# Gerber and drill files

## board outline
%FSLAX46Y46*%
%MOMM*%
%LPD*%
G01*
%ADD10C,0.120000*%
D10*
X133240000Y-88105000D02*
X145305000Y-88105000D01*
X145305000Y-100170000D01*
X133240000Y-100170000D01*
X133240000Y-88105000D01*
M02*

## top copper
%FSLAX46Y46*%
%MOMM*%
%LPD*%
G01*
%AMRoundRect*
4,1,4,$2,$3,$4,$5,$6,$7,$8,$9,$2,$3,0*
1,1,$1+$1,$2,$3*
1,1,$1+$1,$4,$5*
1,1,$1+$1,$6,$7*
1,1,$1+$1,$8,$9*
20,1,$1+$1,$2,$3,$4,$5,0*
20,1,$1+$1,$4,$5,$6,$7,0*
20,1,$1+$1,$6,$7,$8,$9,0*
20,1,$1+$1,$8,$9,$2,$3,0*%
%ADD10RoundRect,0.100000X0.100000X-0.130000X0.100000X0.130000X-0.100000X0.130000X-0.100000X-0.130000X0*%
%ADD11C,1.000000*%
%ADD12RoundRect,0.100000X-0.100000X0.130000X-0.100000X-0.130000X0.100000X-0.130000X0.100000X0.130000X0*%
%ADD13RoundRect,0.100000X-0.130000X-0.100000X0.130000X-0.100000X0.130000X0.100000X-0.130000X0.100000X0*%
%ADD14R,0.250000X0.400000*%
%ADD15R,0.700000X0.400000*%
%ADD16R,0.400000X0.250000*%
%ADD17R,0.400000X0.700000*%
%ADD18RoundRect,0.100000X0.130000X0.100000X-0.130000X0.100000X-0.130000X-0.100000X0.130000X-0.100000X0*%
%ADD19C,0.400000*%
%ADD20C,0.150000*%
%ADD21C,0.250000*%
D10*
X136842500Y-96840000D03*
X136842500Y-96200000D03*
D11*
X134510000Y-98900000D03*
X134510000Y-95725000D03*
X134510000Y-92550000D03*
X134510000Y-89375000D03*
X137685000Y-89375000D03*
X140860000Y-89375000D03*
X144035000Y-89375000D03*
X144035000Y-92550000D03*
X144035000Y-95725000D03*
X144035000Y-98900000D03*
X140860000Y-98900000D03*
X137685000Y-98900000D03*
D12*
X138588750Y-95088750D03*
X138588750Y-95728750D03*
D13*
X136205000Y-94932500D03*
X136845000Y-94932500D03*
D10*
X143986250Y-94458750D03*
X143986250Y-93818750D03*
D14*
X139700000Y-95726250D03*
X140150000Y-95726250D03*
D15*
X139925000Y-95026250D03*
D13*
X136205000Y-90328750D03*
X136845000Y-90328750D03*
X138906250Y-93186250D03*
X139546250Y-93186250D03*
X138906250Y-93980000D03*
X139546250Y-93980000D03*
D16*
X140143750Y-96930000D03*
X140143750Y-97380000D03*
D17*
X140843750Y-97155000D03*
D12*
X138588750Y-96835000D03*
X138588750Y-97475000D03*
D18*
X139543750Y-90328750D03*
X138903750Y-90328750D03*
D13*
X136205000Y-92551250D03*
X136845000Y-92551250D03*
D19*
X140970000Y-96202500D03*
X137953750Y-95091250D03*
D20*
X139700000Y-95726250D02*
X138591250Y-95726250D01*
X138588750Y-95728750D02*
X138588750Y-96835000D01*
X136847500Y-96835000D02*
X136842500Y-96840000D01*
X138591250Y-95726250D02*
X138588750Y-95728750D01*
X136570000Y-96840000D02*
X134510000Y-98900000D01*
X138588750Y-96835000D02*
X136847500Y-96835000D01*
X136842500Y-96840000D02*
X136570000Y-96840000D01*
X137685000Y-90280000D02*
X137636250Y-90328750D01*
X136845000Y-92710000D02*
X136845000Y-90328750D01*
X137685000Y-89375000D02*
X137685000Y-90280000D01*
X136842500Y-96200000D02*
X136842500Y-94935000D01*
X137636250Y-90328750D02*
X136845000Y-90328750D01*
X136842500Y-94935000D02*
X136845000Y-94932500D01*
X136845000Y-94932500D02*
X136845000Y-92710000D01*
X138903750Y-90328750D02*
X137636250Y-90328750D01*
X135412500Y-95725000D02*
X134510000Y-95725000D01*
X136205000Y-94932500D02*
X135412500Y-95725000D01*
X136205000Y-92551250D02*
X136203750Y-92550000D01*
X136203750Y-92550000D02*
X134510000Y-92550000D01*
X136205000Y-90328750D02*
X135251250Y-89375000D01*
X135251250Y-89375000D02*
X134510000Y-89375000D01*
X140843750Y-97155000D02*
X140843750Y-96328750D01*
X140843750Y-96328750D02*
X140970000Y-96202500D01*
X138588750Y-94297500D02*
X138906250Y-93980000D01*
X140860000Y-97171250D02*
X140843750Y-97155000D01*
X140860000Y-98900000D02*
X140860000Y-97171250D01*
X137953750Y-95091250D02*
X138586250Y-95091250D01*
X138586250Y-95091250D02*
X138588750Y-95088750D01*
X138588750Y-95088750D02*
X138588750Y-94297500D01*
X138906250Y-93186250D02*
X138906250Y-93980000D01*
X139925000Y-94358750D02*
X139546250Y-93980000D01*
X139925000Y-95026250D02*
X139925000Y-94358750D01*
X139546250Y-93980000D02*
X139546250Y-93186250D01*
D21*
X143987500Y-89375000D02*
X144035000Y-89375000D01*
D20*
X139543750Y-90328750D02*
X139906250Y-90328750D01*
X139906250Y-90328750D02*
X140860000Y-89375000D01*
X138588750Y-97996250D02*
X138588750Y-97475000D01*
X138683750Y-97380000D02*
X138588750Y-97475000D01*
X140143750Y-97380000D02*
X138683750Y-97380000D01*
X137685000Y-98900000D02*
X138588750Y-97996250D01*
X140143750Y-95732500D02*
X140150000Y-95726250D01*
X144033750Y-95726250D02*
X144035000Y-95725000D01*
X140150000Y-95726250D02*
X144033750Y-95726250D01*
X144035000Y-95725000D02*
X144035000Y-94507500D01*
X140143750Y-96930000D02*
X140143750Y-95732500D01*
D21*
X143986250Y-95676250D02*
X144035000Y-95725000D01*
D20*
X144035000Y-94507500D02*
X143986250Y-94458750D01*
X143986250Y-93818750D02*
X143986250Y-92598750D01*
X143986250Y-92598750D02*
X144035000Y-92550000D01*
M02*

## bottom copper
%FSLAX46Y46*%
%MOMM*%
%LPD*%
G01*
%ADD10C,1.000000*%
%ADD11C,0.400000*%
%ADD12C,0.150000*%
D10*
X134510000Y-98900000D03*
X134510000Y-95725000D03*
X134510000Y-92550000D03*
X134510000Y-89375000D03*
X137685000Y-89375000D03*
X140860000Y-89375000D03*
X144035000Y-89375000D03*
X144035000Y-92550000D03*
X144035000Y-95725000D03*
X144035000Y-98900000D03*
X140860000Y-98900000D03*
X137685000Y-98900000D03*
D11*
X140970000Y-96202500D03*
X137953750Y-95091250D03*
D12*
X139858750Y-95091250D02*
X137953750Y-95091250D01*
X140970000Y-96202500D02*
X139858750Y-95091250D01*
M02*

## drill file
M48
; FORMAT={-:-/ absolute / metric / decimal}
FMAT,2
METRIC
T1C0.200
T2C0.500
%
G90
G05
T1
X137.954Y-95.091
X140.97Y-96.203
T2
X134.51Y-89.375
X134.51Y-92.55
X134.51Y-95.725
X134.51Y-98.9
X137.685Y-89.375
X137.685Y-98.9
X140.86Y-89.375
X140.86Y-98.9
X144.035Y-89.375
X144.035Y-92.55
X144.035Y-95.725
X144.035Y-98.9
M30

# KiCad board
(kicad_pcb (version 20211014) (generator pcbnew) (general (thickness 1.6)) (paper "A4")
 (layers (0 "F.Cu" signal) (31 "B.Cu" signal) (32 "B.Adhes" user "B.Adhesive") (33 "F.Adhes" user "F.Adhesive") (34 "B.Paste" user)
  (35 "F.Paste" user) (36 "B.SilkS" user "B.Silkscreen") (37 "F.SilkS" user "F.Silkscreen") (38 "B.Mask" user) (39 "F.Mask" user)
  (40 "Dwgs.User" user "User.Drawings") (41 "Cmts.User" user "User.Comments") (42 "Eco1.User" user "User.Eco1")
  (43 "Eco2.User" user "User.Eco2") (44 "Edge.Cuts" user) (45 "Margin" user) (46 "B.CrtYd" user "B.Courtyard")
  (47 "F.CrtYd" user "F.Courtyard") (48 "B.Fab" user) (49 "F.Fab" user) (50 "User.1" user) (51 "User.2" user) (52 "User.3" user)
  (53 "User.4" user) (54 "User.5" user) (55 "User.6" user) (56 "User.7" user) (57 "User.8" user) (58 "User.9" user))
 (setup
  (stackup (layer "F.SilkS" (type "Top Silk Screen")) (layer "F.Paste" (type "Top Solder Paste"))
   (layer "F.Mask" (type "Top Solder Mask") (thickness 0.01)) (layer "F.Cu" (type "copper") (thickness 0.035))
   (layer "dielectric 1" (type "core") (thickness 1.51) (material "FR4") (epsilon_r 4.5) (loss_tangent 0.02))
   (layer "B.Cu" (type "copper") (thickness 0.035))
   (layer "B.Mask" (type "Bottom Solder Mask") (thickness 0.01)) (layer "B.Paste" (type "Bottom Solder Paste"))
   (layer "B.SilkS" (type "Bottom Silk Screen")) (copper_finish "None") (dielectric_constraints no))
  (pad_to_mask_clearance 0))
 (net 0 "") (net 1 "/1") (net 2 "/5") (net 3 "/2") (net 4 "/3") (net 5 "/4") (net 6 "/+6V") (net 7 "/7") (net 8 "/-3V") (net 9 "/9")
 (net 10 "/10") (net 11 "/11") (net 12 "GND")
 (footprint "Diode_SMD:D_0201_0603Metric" (layer "F.Cu") (at 136.8425 96.52 90)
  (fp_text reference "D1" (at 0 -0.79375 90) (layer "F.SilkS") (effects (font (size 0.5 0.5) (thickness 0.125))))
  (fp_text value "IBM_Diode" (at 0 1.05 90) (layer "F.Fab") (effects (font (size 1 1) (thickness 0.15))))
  (pad "" smd roundrect locked (at -0.345 0 90) (size 0.318 0.36) (layers "F.Paste") (roundrect_rratio 0.25))
  (pad "" smd roundrect locked (at 0.345 0 90) (size 0.318 0.36) (layers "F.Paste") (roundrect_rratio 0.25))
  (pad "1" smd roundrect locked (at -0.32 0 90) (size 0.46 0.4) (layers "F.Cu" "F.Mask") (roundrect_rratio 0.25) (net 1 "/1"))
  (pad "2" smd roundrect locked (at 0.32 0 90) (size 0.46 0.4) (layers "F.Cu" "F.Mask") (roundrect_rratio 0.25) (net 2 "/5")))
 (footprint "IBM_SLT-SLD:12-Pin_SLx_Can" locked (layer "F.Cu") (at 134.51 98.9)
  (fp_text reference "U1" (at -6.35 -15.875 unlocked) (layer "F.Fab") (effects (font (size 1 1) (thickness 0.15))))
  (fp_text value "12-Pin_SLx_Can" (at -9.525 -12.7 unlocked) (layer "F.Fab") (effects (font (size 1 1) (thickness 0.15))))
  (fp_rect (start -1.27 -10.795) (end 10.795 1.27) (layer "Edge.Cuts") (width 0.12) (fill none))
  (pad "1" thru_hole circle locked (at 0 0) (size 1 1) (drill 0.5) (layers *.Cu *.Mask) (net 1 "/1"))
  (pad "2" thru_hole circle locked (at 0 -3.175) (size 1 1) (drill 0.5) (layers *.Cu *.Mask) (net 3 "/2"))
  (pad "3" thru_hole circle locked (at 0 -6.35) (size 1 1) (drill 0.5) (layers *.Cu *.Mask) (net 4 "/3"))
  (pad "4" thru_hole circle locked (at 0 -9.525) (size 1 1) (drill 0.5) (layers *.Cu *.Mask) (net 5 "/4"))
  (pad "5" thru_hole circle locked (at 3.175 -9.525) (size 1 1) (drill 0.5) (layers *.Cu *.Mask) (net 2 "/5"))
  (pad "6" thru_hole circle locked (at 6.35 -9.525) (size 1 1) (drill 0.5) (layers *.Cu *.Mask) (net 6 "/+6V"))
  (pad "7" thru_hole circle locked (at 9.525 -9.525) (size 1 1) (drill 0.5) (layers *.Cu *.Mask) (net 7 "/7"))
  (pad "8" thru_hole circle locked (at 9.525 -6.35) (size 1 1) (drill 0.5) (layers *.Cu *.Mask) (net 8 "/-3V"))
  (pad "9" thru_hole circle locked (at 9.525 -3.175) (size 1 1) (drill 0.5) (layers *.Cu *.Mask) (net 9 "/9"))
  (pad "10" thru_hole circle locked (at 9.525 0) (size 1 1) (drill 0.5) (layers *.Cu *.Mask) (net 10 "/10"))
  (pad "11" thru_hole circle locked (at 6.35 0) (size 1 1) (drill 0.5) (layers *.Cu *.Mask) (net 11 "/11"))
  (pad "12" thru_hole circle locked (at 3.175 0) (size 1 1) (drill 0.5) (layers *.Cu *.Mask) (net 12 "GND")))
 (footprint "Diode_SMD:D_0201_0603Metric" (layer "F.Cu") (at 138.58875 95.40875 -90)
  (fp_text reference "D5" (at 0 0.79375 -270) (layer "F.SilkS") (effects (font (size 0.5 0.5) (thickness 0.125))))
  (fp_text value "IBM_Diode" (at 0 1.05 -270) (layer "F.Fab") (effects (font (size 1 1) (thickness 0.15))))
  (pad "" smd roundrect locked (at 0.345 0 270) (size 0.318 0.36) (layers "F.Paste") (roundrect_rratio 0.25))
  (pad "" smd roundrect locked (at -0.345 0 270) (size 0.318 0.36) (layers "F.Paste") (roundrect_rratio 0.25))
  (pad "1" smd roundrect locked (at -0.32 0 270) (size 0.46 0.4) (layers "F.Cu" "F.Mask") (roundrect_rratio 0.25) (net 11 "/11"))
  (pad "2" smd roundrect locked (at 0.32 0 270) (size 0.46 0.4) (layers "F.Cu" "F.Mask") (roundrect_rratio 0.25) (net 1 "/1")))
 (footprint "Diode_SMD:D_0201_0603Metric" (layer "F.Cu") (at 136.525 94.9325)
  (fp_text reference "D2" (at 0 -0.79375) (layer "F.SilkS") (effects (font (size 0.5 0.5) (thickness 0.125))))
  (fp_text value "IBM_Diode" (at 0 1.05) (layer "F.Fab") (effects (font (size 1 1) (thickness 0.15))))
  (pad "" smd roundrect locked (at -0.345 0) (size 0.318 0.36) (layers "F.Paste") (roundrect_rratio 0.25))
  (pad "" smd roundrect locked (at 0.345 0) (size 0.318 0.36) (layers "F.Paste") (roundrect_rratio 0.25))
  (pad "1" smd roundrect locked (at -0.32 0) (size 0.46 0.4) (layers "F.Cu" "F.Mask") (roundrect_rratio 0.25) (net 3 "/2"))
  (pad "2" smd roundrect locked (at 0.32 0) (size 0.46 0.4) (layers "F.Cu" "F.Mask") (roundrect_rratio 0.25) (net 2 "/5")))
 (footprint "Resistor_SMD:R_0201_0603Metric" (layer "F.Cu") (at 143.98625 94.13875 90)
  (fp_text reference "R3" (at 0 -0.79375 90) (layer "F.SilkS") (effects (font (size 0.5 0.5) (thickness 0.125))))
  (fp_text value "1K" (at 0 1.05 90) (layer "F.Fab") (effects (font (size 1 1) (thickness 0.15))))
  (pad "" smd roundrect locked (at -0.345 0 90) (size 0.318 0.36) (layers "F.Paste") (roundrect_rratio 0.25))
  (pad "" smd roundrect locked (at 0.345 0 90) (size 0.318 0.36) (layers "F.Paste") (roundrect_rratio 0.25))
  (pad "1" smd roundrect locked (at -0.32 0 90) (size 0.46 0.4) (layers "F.Cu" "F.Mask") (roundrect_rratio 0.25) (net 9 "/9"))
  (pad "2" smd roundrect locked (at 0.32 0 90) (size 0.46 0.4) (layers "F.Cu" "F.Mask") (roundrect_rratio 0.25) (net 8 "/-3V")))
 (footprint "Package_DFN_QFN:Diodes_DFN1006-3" (layer "F.Cu") (at 139.925 95.37625 90)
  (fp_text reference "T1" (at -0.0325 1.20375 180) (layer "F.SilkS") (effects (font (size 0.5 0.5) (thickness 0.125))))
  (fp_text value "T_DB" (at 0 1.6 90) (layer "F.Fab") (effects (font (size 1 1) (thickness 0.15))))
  (pad "1" smd rect locked (at -0.35 -0.225) (size 0.25 0.4) (layers "F.Cu" "F.Paste" "F.Mask") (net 1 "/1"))
  (pad "2" smd rect locked (at -0.35 0.225) (size 0.25 0.4) (layers "F.Cu" "F.Paste" "F.Mask") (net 9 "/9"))
  (pad "3" smd rect locked (at 0.35 0) (size 0.7 0.4) (layers "F.Cu" "F.Paste" "F.Mask") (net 7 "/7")))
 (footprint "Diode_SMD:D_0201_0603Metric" (layer "F.Cu") (at 136.525 90.32875)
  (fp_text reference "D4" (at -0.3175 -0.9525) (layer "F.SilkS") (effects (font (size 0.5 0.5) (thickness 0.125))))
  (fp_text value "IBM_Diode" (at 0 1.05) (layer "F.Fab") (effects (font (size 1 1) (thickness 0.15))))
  (pad "" smd roundrect locked (at 0.345 0) (size 0.318 0.36) (layers "F.Paste") (roundrect_rratio 0.25))
  (pad "" smd roundrect locked (at -0.345 0) (size 0.318 0.36) (layers "F.Paste") (roundrect_rratio 0.25))
  (pad "1" smd roundrect locked (at -0.32 0) (size 0.46 0.4) (layers "F.Cu" "F.Mask") (roundrect_rratio 0.25) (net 5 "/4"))
  (pad "2" smd roundrect locked (at 0.32 0) (size 0.46 0.4) (layers "F.Cu" "F.Mask") (roundrect_rratio 0.25) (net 2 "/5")))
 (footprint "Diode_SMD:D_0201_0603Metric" (layer "F.Cu") (at 139.22625 93.18625)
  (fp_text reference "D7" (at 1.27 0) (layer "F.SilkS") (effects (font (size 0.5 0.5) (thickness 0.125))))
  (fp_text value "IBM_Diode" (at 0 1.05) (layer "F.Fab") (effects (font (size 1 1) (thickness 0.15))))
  (pad "" smd roundrect locked (at -0.345 0) (size 0.318 0.36) (layers "F.Paste") (roundrect_rratio 0.25))
  (pad "" smd roundrect locked (at 0.345 0) (size 0.318 0.36) (layers "F.Paste") (roundrect_rratio 0.25))
  (pad "1" smd roundrect locked (at -0.32 0) (size 0.46 0.4) (layers "F.Cu" "F.Mask") (roundrect_rratio 0.25) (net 11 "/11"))
  (pad "2" smd roundrect locked (at 0.32 0) (size 0.46 0.4) (layers "F.Cu" "F.Mask") (roundrect_rratio 0.25) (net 7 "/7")))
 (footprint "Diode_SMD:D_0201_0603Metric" (layer "F.Cu") (at 139.22625 93.98)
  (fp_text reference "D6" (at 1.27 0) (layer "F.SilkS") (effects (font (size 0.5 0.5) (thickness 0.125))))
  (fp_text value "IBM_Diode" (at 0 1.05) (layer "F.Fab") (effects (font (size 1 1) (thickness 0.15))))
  (pad "" smd roundrect locked (at 0.345 0) (size 0.318 0.36) (layers "F.Paste") (roundrect_rratio 0.25))
  (pad "" smd roundrect locked (at -0.345 0) (size 0.318 0.36) (layers "F.Paste") (roundrect_rratio 0.25))
  (pad "1" smd roundrect locked (at -0.32 0) (size 0.46 0.4) (layers "F.Cu" "F.Mask") (roundrect_rratio 0.25) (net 11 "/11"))
  (pad "2" smd roundrect locked (at 0.32 0) (size 0.46 0.4) (layers "F.Cu" "F.Mask") (roundrect_rratio 0.25) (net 7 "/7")))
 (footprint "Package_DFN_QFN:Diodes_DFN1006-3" (layer "F.Cu") (at 140.49375 97.155)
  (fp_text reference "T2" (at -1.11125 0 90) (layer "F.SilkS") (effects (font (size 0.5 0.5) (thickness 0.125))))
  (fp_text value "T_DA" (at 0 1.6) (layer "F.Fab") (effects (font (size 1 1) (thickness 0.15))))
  (pad "1" smd rect locked (at -0.35 -0.225 270) (size 0.25 0.4) (layers "F.Cu" "F.Paste" "F.Mask") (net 9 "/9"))
  (pad "2" smd rect locked (at -0.35 0.225 270) (size 0.25 0.4) (layers "F.Cu" "F.Paste" "F.Mask") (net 12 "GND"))
  (pad "3" smd rect locked (at 0.35 0 270) (size 0.7 0.4) (layers "F.Cu" "F.Paste" "F.Mask") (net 11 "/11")))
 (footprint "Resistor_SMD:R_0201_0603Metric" (layer "F.Cu") (at 138.58875 97.155 -90)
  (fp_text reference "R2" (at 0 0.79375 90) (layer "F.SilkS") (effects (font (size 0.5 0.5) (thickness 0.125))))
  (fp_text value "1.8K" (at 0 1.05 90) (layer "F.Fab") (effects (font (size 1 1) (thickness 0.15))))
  (pad "" smd roundrect locked (at -0.345 0 270) (size 0.318 0.36) (layers "F.Paste") (roundrect_rratio 0.25))
  (pad "" smd roundrect locked (at 0.345 0 270) (size 0.318 0.36) (layers "F.Paste") (roundrect_rratio 0.25))
  (pad "1" smd roundrect locked (at -0.32 0 270) (size 0.46 0.4) (layers "F.Cu" "F.Mask") (roundrect_rratio 0.25) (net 1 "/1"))
  (pad "2" smd roundrect locked (at 0.32 0 270) (size 0.46 0.4) (layers "F.Cu" "F.Mask") (roundrect_rratio 0.25) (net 12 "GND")))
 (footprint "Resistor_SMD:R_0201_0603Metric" (layer "F.Cu") (at 139.22375 90.32875 180)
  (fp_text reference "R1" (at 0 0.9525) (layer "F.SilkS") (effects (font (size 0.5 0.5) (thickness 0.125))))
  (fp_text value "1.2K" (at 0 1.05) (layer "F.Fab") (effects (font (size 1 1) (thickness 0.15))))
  (pad "" smd roundrect locked (at 0.345 0 180) (size 0.318 0.36) (layers "F.Paste") (roundrect_rratio 0.25))
  (pad "" smd roundrect locked (at -0.345 0 180) (size 0.318 0.36) (layers "F.Paste") (roundrect_rratio 0.25))
  (pad "1" smd roundrect locked (at -0.32 0 180) (size 0.46 0.4) (layers "F.Cu" "F.Mask") (roundrect_rratio 0.25) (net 6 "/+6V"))
  (pad "2" smd roundrect locked (at 0.32 0 180) (size 0.46 0.4) (layers "F.Cu" "F.Mask") (roundrect_rratio 0.25) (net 2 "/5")))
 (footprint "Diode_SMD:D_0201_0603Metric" (layer "F.Cu") (at 136.525 92.55125)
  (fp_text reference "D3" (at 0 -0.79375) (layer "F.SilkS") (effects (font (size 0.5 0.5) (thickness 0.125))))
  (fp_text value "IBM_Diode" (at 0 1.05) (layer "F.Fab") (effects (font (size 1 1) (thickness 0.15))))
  (pad "" smd roundrect locked (at -0.345 0) (size 0.318 0.36) (layers "F.Paste") (roundrect_rratio 0.25))
  (pad "" smd roundrect locked (at 0.345 0) (size 0.318 0.36) (layers "F.Paste") (roundrect_rratio 0.25))
  (pad "1" smd roundrect locked (at -0.32 0) (size 0.46 0.4) (layers "F.Cu" "F.Mask") (roundrect_rratio 0.25) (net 4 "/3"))
  (pad "2" smd roundrect locked (at 0.32 0) (size 0.46 0.4) (layers "F.Cu" "F.Mask") (roundrect_rratio 0.25) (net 2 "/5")))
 (segment (start 139.7 95.72625) (end 138.59125 95.72625) (width 0.15) (layer "F.Cu") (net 1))
 (segment (start 138.58875 95.72875) (end 138.58875 96.835) (width 0.15) (layer "F.Cu") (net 1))
 (segment (start 136.8475 96.835) (end 136.8425 96.84) (width 0.15) (layer "F.Cu") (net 1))
 (segment (start 138.59125 95.72625) (end 138.58875 95.72875) (width 0.15) (layer "F.Cu") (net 1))
 (segment (start 136.57 96.84) (end 134.51 98.9) (width 0.15) (layer "F.Cu") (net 1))
 (segment (start 138.58875 96.835) (end 136.8475 96.835) (width 0.15) (layer "F.Cu") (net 1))
 (segment (start 136.8425 96.84) (end 136.57 96.84) (width 0.15) (layer "F.Cu") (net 1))
 (segment (start 137.685 90.28) (end 137.63625 90.32875) (width 0.15) (layer "F.Cu") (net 2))
 (segment (start 136.845 92.71) (end 136.845 90.32875) (width 0.15) (layer "F.Cu") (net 2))
 (segment (start 137.685 89.375) (end 137.685 90.28) (width 0.15) (layer "F.Cu") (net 2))
 (segment (start 136.8425 96.2) (end 136.8425 94.935) (width 0.15) (layer "F.Cu") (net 2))
 (segment (start 137.63625 90.32875) (end 136.845 90.32875) (width 0.15) (layer "F.Cu") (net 2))
 (segment (start 136.8425 94.935) (end 136.845 94.9325) (width 0.15) (layer "F.Cu") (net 2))
 (segment (start 136.845 94.9325) (end 136.845 92.71) (width 0.15) (layer "F.Cu") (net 2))
 (segment (start 138.90375 90.32875) (end 137.63625 90.32875) (width 0.15) (layer "F.Cu") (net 2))
 (segment (start 135.4125 95.725) (end 134.51 95.725) (width 0.15) (layer "F.Cu") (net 3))
 (segment (start 136.205 94.9325) (end 135.4125 95.725) (width 0.15) (layer "F.Cu") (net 3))
 (segment (start 136.205 92.55125) (end 136.20375 92.55) (width 0.15) (layer "F.Cu") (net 4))
 (segment (start 136.20375 92.55) (end 134.51 92.55) (width 0.15) (layer "F.Cu") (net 4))
 (segment (start 136.205 90.32875) (end 135.25125 89.375) (width 0.15) (layer "F.Cu") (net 5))
 (segment (start 135.25125 89.375) (end 134.51 89.375) (width 0.15) (layer "F.Cu") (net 5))
 (segment (start 140.84375 97.155) (end 140.84375 96.32875) (width 0.15) (layer "F.Cu") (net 11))
 (segment (start 140.84375 96.32875) (end 140.97 96.2025) (width 0.15) (layer "F.Cu") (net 11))
 (segment (start 138.58875 94.2975) (end 138.90625 93.98) (width 0.15) (layer "F.Cu") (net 11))
 (segment (start 140.86 97.17125) (end 140.84375 97.155) (width 0.15) (layer "F.Cu") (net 11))
 (segment (start 140.86 98.9) (end 140.86 97.17125) (width 0.15) (layer "F.Cu") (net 11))
 (segment (start 137.95375 95.09125) (end 138.58625 95.09125) (width 0.15) (layer "F.Cu") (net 11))
 (segment (start 138.58625 95.09125) (end 138.58875 95.08875) (width 0.15) (layer "F.Cu") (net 11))
 (segment (start 138.58875 95.08875) (end 138.58875 94.2975) (width 0.15) (layer "F.Cu") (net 11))
 (segment (start 138.90625 93.18625) (end 138.90625 93.98) (width 0.15) (layer "F.Cu") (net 11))
 (via (at 140.97 96.2025) (size 0.4) (drill 0.2) (layers "F.Cu" "B.Cu") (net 11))
 (via (at 137.95375 95.09125) (size 0.4) (drill 0.2) (layers "F.Cu" "B.Cu") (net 11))
 (segment (start 139.85875 95.09125) (end 137.95375 95.09125) (width 0.15) (layer "B.Cu") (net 11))
 (segment (start 140.97 96.2025) (end 139.85875 95.09125) (width 0.15) (layer "B.Cu") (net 11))
 (segment (start 139.925 94.35875) (end 139.54625 93.98) (width 0.15) (layer "F.Cu") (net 7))
 (segment (start 139.925 95.02625) (end 139.925 94.35875) (width 0.15) (layer "F.Cu") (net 7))
 (segment (start 139.54625 93.98) (end 139.54625 93.18625) (width 0.15) (layer "F.Cu") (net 7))
 (segment (start 143.9875 89.375) (end 144.035 89.375) (width 0.25) (layer "F.Cu") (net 7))
 (segment (start 139.54375 90.32875) (end 139.90625 90.32875) (width 0.15) (layer "F.Cu") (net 6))
 (segment (start 139.90625 90.32875) (end 140.86 89.375) (width 0.15) (layer "F.Cu") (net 6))
 (segment (start 138.58875 97.99625) (end 138.58875 97.475) (width 0.15) (layer "F.Cu") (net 12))
 (segment (start 138.68375 97.38) (end 138.58875 97.475) (width 0.15) (layer "F.Cu") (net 12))
 (segment (start 140.14375 97.38) (end 138.68375 97.38) (width 0.15) (layer "F.Cu") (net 12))
 (segment (start 137.685 98.9) (end 138.58875 97.99625) (width 0.15) (layer "F.Cu") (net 12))
 (segment (start 140.14375 95.7325) (end 140.15 95.72625) (width 0.15) (layer "F.Cu") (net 9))
 (segment (start 144.03375 95.72625) (end 144.035 95.725) (width 0.15) (layer "F.Cu") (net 9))
 (segment (start 140.15 95.72625) (end 144.03375 95.72625) (width 0.15) (layer "F.Cu") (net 9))
 (segment (start 144.035 95.725) (end 144.035 94.5075) (width 0.15) (layer "F.Cu") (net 9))
 (segment (start 140.14375 96.93) (end 140.14375 95.7325) (width 0.15) (layer "F.Cu") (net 9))
 (segment (start 143.98625 95.67625) (end 144.035 95.725) (width 0.25) (layer "F.Cu") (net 9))
 (segment (start 144.035 94.5075) (end 143.98625 94.45875) (width 0.15) (layer "F.Cu") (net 9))
 (segment (start 143.98625 93.81875) (end 143.98625 92.59875) (width 0.15) (layer "F.Cu") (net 8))
 (segment (start 143.98625 92.59875) (end 144.035 92.55) (width 0.15) (layer "F.Cu") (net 8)))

